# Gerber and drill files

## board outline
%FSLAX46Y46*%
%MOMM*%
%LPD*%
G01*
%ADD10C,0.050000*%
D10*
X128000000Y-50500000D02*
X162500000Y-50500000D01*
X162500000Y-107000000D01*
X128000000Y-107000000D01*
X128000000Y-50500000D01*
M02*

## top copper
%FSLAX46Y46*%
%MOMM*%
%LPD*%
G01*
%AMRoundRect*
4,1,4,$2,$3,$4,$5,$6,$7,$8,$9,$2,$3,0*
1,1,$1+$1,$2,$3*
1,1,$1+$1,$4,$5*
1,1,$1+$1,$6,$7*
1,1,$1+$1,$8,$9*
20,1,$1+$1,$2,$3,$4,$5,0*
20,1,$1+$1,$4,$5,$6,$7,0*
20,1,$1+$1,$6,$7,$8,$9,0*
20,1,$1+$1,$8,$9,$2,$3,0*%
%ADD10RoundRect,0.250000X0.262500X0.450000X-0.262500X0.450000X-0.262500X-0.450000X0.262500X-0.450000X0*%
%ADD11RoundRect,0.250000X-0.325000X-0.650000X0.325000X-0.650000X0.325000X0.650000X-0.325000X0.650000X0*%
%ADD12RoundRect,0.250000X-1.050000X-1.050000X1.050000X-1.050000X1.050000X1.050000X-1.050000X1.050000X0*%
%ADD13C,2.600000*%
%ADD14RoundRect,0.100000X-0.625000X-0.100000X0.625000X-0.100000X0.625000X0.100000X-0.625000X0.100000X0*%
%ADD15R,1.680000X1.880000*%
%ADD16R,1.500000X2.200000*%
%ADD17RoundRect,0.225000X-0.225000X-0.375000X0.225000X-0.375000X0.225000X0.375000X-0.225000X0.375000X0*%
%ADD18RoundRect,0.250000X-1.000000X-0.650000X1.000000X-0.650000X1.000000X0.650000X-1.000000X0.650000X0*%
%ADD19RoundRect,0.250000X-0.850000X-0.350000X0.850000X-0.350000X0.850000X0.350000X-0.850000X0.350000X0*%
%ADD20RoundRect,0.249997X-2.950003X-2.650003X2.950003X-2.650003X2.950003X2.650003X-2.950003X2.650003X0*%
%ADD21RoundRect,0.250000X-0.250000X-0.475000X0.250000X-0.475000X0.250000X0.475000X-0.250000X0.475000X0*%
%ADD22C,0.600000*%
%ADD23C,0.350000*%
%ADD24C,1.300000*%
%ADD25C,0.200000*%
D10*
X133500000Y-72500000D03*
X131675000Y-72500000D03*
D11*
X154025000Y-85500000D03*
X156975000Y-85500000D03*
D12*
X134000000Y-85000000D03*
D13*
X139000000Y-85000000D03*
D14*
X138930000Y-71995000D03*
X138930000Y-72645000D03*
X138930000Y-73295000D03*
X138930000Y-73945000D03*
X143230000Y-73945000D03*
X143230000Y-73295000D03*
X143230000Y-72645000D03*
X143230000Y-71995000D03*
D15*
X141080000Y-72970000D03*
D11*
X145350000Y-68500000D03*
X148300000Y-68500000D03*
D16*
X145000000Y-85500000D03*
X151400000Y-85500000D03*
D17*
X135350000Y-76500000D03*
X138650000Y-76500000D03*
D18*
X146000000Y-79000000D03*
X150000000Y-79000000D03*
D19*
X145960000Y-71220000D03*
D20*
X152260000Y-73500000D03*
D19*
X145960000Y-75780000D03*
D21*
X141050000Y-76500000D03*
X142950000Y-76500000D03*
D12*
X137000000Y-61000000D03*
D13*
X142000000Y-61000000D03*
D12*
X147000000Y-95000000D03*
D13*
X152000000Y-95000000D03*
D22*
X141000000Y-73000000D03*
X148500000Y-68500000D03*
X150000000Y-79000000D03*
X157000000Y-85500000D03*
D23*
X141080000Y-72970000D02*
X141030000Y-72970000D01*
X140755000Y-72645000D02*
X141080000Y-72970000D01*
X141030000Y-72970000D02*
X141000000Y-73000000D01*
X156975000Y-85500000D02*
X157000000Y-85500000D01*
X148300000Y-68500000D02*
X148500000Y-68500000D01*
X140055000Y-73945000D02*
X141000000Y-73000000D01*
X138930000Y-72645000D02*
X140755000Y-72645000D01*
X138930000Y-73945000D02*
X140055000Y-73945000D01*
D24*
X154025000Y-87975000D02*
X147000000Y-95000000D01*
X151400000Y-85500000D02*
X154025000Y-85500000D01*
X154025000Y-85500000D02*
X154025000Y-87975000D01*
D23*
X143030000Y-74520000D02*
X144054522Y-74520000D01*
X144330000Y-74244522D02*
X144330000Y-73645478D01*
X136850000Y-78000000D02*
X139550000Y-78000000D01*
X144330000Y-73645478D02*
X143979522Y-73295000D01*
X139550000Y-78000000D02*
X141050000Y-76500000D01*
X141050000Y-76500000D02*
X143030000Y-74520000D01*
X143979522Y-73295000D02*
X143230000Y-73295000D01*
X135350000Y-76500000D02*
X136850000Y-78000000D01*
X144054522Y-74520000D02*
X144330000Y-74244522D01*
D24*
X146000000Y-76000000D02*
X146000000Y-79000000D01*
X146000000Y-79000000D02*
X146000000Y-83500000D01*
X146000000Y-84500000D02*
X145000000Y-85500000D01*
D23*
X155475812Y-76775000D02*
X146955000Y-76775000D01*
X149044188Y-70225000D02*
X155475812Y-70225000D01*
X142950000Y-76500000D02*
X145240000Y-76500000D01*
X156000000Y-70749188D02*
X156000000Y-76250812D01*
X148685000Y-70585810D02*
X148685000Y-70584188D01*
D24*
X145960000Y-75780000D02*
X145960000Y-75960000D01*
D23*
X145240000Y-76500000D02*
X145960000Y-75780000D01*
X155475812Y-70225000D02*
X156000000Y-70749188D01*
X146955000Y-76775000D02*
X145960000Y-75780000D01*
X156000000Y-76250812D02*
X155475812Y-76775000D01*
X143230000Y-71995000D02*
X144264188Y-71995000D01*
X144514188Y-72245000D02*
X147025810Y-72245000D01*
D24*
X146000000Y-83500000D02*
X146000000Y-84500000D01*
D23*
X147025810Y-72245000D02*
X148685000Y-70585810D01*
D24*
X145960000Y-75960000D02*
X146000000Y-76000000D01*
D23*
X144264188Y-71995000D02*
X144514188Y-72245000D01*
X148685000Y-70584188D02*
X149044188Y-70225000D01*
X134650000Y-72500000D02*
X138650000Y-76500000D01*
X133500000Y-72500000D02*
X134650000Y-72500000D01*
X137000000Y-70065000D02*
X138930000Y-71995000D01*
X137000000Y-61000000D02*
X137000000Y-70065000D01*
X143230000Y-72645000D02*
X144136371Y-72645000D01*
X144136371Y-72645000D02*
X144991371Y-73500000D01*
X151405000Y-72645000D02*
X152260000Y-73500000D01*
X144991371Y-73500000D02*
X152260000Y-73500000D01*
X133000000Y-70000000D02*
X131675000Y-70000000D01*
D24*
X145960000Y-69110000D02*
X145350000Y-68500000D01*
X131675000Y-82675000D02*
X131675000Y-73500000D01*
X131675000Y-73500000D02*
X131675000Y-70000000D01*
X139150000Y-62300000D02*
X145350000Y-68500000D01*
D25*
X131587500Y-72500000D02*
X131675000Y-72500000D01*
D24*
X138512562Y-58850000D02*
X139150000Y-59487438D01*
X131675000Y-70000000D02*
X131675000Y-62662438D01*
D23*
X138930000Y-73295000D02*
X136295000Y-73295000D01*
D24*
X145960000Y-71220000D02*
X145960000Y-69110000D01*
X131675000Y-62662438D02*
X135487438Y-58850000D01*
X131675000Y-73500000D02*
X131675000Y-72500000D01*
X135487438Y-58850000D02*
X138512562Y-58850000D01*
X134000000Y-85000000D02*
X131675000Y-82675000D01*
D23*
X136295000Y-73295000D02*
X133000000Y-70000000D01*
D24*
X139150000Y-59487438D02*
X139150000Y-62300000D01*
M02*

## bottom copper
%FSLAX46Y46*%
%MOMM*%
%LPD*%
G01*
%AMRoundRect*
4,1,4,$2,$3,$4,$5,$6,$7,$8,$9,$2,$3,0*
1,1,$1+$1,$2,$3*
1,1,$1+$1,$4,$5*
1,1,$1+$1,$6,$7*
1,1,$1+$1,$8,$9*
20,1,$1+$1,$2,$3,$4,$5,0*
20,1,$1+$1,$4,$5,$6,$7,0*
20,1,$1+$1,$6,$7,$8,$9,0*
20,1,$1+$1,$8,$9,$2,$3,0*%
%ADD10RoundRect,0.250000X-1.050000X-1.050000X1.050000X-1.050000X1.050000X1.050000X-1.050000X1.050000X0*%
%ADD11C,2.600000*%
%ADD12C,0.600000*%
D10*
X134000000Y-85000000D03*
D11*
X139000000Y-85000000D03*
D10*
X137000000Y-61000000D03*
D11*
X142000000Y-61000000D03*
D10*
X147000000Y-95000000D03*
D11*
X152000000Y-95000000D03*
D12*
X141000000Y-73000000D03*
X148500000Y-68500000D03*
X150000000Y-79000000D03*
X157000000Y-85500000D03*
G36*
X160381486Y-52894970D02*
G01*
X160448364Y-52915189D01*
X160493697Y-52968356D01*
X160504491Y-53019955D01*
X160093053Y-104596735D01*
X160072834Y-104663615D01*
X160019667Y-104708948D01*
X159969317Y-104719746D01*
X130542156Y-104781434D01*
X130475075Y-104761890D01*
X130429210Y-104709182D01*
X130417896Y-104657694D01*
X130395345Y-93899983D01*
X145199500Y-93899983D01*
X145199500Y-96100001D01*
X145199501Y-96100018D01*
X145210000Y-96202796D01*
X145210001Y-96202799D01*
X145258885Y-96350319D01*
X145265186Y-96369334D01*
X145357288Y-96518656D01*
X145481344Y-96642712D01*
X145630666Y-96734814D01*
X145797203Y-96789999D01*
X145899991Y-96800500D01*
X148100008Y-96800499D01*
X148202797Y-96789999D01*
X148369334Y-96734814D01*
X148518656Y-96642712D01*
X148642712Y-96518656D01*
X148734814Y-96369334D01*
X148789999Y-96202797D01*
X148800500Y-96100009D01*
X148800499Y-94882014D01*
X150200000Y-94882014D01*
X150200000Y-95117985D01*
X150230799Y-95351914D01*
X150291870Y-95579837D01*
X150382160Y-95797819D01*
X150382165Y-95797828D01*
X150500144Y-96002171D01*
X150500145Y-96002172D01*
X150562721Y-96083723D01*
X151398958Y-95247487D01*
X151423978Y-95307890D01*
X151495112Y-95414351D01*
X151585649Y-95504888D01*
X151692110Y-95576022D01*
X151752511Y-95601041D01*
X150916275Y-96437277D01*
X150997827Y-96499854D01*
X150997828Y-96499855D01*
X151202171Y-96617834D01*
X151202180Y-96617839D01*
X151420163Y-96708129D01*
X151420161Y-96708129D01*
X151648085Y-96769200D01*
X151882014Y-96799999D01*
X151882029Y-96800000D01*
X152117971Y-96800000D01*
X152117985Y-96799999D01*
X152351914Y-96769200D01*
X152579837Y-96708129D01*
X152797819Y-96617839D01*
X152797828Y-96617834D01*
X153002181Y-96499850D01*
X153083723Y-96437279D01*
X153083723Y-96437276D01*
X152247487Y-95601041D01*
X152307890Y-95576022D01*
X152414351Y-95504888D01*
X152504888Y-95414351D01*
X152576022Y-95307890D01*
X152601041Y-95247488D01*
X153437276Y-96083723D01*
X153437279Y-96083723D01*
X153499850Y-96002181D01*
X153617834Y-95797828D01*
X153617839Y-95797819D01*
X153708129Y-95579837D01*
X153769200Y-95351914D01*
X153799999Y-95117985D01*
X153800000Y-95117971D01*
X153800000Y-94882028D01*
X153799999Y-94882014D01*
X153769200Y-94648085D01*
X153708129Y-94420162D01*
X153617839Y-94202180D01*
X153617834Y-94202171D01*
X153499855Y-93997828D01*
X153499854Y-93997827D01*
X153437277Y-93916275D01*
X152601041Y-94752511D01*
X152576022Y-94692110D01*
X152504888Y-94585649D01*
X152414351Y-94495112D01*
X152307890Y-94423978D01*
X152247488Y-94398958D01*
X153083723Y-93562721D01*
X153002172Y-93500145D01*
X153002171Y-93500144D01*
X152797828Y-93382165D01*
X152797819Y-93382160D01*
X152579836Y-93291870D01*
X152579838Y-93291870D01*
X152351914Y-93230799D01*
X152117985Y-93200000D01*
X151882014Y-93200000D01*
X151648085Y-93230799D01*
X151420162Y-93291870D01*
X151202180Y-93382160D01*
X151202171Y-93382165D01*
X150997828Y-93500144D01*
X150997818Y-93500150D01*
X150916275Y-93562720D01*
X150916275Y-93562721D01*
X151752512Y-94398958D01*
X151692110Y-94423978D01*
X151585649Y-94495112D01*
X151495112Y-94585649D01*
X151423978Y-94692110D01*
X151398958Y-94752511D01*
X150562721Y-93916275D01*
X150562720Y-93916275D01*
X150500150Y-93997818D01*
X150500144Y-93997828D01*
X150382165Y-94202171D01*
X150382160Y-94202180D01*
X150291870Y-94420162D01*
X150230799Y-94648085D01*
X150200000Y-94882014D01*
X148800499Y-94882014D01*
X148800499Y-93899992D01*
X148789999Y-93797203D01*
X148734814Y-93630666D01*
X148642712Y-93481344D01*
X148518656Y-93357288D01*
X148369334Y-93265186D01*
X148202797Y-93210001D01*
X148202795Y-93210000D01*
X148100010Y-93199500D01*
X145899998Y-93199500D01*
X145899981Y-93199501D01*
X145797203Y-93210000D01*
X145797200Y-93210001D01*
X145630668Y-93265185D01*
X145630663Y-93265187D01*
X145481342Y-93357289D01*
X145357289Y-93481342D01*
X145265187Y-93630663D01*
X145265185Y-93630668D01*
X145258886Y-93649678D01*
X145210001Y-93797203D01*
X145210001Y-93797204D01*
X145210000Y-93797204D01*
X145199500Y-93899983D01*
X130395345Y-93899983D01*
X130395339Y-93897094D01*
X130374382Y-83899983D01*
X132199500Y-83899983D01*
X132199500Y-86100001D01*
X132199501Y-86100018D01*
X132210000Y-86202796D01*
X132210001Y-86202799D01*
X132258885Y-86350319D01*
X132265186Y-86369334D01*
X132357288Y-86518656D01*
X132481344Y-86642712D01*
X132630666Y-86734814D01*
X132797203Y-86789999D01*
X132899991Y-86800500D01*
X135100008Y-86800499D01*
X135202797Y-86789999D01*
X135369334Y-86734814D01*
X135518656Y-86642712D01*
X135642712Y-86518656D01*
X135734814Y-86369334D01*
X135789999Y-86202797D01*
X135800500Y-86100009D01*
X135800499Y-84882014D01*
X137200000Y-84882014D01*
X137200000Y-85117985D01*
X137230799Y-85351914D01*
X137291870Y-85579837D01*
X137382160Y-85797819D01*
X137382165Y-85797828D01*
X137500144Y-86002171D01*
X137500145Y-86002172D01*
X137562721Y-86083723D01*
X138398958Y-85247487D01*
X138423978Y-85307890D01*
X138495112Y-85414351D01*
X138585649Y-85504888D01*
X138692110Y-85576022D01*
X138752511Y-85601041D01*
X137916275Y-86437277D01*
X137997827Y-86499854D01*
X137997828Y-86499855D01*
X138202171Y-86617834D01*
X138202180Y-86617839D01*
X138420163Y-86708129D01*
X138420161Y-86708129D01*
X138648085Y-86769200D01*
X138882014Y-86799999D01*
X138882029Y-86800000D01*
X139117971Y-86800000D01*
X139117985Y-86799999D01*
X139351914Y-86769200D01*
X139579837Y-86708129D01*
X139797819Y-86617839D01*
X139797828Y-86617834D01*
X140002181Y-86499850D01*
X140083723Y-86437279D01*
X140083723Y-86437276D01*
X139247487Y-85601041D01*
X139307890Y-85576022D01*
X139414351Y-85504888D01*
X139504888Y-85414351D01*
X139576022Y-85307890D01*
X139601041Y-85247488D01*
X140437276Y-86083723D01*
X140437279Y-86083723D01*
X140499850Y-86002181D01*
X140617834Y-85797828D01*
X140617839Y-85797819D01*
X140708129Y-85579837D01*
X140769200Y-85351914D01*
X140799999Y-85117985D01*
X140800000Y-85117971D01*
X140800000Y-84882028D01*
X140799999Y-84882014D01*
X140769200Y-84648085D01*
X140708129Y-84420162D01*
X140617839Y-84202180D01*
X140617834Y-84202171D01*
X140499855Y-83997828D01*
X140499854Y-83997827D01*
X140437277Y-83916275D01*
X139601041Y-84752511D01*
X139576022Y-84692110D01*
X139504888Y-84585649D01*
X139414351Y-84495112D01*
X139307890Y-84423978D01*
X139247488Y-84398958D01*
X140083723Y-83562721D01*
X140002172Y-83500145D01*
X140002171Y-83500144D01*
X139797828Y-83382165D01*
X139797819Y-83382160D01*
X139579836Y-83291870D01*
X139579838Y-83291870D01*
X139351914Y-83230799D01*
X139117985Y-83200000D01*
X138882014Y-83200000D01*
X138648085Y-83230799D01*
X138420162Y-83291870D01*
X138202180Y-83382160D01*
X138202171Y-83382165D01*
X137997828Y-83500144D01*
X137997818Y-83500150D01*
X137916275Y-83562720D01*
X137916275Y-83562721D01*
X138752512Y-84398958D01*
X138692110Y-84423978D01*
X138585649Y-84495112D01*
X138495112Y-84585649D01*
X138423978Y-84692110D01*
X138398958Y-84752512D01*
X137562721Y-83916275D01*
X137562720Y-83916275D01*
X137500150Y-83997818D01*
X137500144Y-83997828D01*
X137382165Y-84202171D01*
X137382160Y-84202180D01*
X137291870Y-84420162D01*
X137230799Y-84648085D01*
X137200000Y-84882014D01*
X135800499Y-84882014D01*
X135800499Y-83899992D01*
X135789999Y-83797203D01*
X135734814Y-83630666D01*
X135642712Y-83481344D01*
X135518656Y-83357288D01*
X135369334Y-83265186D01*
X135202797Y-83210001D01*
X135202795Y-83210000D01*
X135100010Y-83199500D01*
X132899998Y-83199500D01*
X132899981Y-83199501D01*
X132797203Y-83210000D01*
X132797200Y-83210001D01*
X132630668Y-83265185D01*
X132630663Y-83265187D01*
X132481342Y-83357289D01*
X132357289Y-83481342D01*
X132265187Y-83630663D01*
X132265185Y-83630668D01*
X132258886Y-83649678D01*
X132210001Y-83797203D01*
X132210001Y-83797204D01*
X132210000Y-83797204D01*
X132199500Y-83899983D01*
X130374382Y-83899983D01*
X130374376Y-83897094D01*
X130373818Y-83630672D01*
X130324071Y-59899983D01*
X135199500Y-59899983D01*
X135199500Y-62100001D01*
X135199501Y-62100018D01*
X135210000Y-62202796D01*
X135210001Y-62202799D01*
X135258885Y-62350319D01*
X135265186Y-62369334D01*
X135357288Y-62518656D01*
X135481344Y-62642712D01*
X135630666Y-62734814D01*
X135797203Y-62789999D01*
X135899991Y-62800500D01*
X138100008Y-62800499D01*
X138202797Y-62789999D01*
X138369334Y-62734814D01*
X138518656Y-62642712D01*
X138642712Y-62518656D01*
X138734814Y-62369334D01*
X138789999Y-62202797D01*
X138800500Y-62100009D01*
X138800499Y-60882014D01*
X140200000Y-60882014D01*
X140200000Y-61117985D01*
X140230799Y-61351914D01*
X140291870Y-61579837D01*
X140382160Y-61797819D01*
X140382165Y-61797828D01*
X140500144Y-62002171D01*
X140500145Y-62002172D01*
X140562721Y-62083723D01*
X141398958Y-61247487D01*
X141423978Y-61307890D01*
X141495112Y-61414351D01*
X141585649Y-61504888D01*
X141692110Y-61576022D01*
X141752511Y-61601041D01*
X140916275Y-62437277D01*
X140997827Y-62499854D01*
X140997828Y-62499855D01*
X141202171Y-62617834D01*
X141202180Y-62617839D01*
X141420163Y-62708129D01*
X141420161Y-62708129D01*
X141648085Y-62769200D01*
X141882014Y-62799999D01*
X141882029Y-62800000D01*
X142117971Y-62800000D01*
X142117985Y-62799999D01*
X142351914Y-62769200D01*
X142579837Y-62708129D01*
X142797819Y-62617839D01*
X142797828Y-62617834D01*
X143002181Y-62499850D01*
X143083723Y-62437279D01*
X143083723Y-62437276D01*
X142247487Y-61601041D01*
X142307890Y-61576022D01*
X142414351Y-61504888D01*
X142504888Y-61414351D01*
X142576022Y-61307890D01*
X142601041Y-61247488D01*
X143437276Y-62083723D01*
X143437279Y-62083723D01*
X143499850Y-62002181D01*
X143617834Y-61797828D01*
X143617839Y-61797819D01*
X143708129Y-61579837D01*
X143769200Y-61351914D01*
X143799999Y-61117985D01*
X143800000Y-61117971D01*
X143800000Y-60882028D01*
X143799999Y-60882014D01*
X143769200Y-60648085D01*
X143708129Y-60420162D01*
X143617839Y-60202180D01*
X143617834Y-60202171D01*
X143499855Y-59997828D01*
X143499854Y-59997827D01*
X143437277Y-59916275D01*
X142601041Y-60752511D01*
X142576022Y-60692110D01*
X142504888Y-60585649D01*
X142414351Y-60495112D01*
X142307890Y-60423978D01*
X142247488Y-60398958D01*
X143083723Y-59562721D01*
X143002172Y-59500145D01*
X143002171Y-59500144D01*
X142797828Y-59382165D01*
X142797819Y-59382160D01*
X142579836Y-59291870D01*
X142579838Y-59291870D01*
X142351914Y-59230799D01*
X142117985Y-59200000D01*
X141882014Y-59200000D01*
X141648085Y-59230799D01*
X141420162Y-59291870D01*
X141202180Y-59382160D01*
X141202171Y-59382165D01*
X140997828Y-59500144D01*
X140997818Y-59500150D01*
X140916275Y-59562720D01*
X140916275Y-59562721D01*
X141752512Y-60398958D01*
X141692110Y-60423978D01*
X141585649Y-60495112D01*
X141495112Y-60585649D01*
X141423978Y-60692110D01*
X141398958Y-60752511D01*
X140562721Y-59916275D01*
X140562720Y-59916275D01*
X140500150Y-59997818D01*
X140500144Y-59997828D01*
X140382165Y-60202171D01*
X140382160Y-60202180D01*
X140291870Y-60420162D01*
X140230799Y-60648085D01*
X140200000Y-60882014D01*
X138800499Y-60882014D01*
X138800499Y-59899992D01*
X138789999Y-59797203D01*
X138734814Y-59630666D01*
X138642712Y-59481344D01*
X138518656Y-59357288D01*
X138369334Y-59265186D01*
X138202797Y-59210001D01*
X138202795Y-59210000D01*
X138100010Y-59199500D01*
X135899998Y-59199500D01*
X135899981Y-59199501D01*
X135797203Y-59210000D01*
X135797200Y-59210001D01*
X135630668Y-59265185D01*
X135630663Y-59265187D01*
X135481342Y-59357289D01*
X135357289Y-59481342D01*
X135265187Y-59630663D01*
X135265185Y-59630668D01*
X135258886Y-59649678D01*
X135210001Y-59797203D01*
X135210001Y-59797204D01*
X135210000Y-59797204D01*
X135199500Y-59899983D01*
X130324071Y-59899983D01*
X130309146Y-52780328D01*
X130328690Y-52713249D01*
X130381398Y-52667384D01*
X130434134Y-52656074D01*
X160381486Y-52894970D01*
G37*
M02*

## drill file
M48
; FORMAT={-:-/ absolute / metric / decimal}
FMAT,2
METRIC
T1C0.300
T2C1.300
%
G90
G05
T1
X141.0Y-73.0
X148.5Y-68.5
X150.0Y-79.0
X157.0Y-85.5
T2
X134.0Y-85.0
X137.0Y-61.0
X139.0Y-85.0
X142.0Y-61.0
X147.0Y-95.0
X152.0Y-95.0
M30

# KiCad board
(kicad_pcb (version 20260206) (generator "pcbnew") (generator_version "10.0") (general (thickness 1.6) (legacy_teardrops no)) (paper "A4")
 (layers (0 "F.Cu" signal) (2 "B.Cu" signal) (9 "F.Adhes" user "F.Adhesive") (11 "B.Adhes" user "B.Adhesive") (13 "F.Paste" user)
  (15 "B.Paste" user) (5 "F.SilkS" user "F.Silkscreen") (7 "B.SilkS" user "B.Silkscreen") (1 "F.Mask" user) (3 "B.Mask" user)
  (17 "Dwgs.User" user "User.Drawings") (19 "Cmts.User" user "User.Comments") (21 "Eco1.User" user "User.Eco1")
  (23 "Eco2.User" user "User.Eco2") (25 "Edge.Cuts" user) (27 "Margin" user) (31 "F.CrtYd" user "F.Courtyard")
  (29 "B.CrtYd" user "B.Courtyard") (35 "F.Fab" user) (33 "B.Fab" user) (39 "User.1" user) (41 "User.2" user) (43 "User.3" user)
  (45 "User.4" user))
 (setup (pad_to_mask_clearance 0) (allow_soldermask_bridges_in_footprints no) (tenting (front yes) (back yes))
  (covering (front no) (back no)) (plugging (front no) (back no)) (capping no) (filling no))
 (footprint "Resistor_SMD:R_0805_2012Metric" (layer "F.Cu") (at 132.5875 72.5 180)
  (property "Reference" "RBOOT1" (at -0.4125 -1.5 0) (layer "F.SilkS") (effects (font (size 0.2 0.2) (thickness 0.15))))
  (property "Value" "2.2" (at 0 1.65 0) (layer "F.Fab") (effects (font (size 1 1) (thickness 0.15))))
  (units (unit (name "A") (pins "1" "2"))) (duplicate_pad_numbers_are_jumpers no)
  (pad "1" smd roundrect (at -0.9125 0 180) (size 1.025 1.4) (layers "F.Cu" "F.Mask" "F.Paste") (roundrect_rratio 0.243902)
   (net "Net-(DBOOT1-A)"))
  (pad "2" smd roundrect (at 0.9125 0 180) (size 1.025 1.4) (layers "F.Cu" "F.Mask" "F.Paste") (roundrect_rratio 0.243902) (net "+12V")))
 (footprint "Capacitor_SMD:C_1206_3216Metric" (layer "F.Cu") (at 155.5 85.5)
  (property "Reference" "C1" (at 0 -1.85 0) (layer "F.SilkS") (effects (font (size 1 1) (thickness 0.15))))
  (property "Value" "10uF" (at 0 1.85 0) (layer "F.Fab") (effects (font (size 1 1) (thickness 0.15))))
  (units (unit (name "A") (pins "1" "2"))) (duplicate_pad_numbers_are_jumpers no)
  (pad "1" smd roundrect (at -1.475 0) (size 1.15 1.8) (layers "F.Cu" "F.Mask" "F.Paste") (roundrect_rratio 0.217391)
   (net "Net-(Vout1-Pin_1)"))
  (pad "2" smd roundrect (at 1.475 0) (size 1.15 1.8) (layers "F.Cu" "F.Mask" "F.Paste") (roundrect_rratio 0.217391) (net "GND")))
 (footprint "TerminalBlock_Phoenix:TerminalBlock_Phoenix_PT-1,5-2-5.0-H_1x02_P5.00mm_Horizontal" (layer "F.Cu") (at 134 85)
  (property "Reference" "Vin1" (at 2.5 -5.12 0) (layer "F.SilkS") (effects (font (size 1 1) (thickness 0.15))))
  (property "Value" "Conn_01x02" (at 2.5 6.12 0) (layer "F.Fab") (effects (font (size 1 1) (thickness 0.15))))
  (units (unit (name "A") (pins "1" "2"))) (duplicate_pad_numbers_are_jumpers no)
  (pad "1" thru_hole roundrect (at 0 0) (size 2.6 2.6) (drill 1.3) (layers "*.Cu" "*.Mask") (remove_unused_layers no)
   (roundrect_rratio 0.096154) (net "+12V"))
  (pad "2" thru_hole circle (at 5 0) (size 2.6 2.6) (drill 1.3) (layers "*.Cu" "*.Mask") (remove_unused_layers no) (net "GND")))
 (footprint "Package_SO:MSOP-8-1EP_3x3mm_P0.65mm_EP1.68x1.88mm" (layer "F.Cu") (at 141.08 72.97)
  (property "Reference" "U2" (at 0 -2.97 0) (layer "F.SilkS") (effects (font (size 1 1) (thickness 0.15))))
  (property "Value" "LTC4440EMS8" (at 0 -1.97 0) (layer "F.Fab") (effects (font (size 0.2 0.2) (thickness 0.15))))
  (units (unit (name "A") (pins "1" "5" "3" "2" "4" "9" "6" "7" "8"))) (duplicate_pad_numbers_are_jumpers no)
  (pad "" smd roundrect (at -0.42 -0.47) (size 0.68 0.76) (layers "F.Paste") (roundrect_rratio 0.25))
  (pad "" smd roundrect (at -0.42 0.47) (size 0.68 0.76) (layers "F.Paste") (roundrect_rratio 0.25))
  (pad "" smd roundrect (at 0.42 -0.47) (size 0.68 0.76) (layers "F.Paste") (roundrect_rratio 0.25))
  (pad "" smd roundrect (at 0.42 0.47) (size 0.68 0.76) (layers "F.Paste") (roundrect_rratio 0.25))
  (pad "1" smd roundrect (at -2.15 -0.975) (size 1.45 0.4) (layers "F.Cu" "F.Mask" "F.Paste") (roundrect_rratio 0.25)
   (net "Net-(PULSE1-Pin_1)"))
  (pad "2" smd roundrect (at -2.15 -0.325) (size 1.45 0.4) (layers "F.Cu" "F.Mask" "F.Paste") (roundrect_rratio 0.25) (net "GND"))
  (pad "3" smd roundrect (at -2.15 0.325) (size 1.45 0.4) (layers "F.Cu" "F.Mask" "F.Paste") (roundrect_rratio 0.25) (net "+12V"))
  (pad "4" smd roundrect (at -2.15 0.975) (size 1.45 0.4) (layers "F.Cu" "F.Mask" "F.Paste") (roundrect_rratio 0.25) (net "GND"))
  (pad "5" smd roundrect (at 2.15 0.975) (size 1.45 0.4) (layers "F.Cu" "F.Mask" "F.Paste") (roundrect_rratio 0.25)
   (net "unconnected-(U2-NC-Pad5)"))
  (pad "6" smd roundrect (at 2.15 0.325) (size 1.45 0.4) (layers "F.Cu" "F.Mask" "F.Paste") (roundrect_rratio 0.25) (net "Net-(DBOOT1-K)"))
  (pad "7" smd roundrect (at 2.15 -0.325) (size 1.45 0.4) (layers "F.Cu" "F.Mask" "F.Paste") (roundrect_rratio 0.25) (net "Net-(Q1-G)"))
  (pad "8" smd roundrect (at 2.15 -0.975) (size 1.45 0.4) (layers "F.Cu" "F.Mask" "F.Paste") (roundrect_rratio 0.25) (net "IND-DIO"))
  (pad "9" smd rect (at 0 0) (size 1.68 1.88) (layers "F.Cu" "F.Mask") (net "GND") (zone_connect 2)))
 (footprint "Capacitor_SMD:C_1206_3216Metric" (layer "F.Cu") (at 146.825 68.5)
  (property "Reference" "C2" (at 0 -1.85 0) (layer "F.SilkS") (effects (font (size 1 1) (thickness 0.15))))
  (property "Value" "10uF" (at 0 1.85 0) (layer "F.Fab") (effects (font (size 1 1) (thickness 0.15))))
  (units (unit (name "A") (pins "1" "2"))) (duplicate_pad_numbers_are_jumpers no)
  (pad "1" smd roundrect (at -1.475 0) (size 1.15 1.8) (layers "F.Cu" "F.Mask" "F.Paste") (roundrect_rratio 0.217391) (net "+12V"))
  (pad "2" smd roundrect (at 1.475 0) (size 1.15 1.8) (layers "F.Cu" "F.Mask" "F.Paste") (roundrect_rratio 0.217391) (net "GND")))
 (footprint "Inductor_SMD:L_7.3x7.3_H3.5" (layer "F.Cu") (at 148.2 85.5)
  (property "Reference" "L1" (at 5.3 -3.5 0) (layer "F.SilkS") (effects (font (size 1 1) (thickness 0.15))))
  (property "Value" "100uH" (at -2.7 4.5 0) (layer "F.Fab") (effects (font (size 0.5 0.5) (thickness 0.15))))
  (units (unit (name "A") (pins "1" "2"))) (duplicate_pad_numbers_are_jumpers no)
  (pad "1" smd rect (at -3.2 0) (size 1.5 2.2) (layers "F.Cu" "F.Mask" "F.Paste") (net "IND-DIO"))
  (pad "2" smd rect (at 3.2 0) (size 1.5 2.2) (layers "F.Cu" "F.Mask" "F.Paste") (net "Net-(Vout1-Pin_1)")))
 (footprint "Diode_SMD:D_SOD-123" (layer "F.Cu") (at 137 76.5)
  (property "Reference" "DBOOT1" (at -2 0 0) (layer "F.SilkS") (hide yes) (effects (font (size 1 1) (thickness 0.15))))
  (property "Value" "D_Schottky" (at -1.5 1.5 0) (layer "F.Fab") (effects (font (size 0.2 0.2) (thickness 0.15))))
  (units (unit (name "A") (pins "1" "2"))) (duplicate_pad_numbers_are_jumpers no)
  (pad "1" smd roundrect (at -1.65 0) (size 0.9 1.2) (layers "F.Cu" "F.Mask" "F.Paste") (roundrect_rratio 0.25) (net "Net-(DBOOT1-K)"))
  (pad "2" smd roundrect (at 1.65 0) (size 0.9 1.2) (layers "F.Cu" "F.Mask" "F.Paste") (roundrect_rratio 0.25) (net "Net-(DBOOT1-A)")))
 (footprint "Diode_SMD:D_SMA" (layer "F.Cu") (at 148 79)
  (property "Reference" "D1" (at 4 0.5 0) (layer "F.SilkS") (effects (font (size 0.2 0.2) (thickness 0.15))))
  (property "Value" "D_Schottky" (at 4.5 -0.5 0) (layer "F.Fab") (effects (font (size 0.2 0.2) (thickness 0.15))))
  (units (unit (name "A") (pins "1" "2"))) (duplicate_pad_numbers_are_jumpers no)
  (pad "1" smd roundrect (at -2 0) (size 2.5 1.8) (layers "F.Cu" "F.Mask" "F.Paste") (roundrect_rratio 0.1388888889) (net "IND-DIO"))
  (pad "2" smd roundrect (at 2 0) (size 2.5 1.8) (layers "F.Cu" "F.Mask" "F.Paste") (roundrect_rratio 0.1388888889) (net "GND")))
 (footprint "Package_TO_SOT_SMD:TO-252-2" (layer "F.Cu") (at 151 73.5)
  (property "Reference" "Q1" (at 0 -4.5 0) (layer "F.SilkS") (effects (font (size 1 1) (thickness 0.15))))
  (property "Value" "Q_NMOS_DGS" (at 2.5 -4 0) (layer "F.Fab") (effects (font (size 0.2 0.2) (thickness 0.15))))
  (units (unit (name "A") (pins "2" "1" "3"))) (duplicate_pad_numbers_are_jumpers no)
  (pad "" smd roundrect (at -0.415 -1.525) (size 3.05 2.75) (layers "F.Paste") (roundrect_rratio 0.090909))
  (pad "" smd roundrect (at -0.415 1.525) (size 3.05 2.75) (layers "F.Paste") (roundrect_rratio 0.090909))
  (pad "" smd roundrect (at 2.935 -1.525) (size 3.05 2.75) (layers "F.Paste") (roundrect_rratio 0.090909))
  (pad "" smd roundrect (at 2.935 1.525) (size 3.05 2.75) (layers "F.Paste") (roundrect_rratio 0.090909))
  (pad "1" smd roundrect (at -5.04 -2.28) (size 2.2 1.2) (layers "F.Cu" "F.Mask" "F.Paste") (roundrect_rratio 0.208333) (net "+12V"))
  (pad "2" smd roundrect (at 1.26 0) (size 6.4 5.8) (layers "F.Cu" "F.Mask") (roundrect_rratio 0.043103) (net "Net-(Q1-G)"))
  (pad "3" smd roundrect (at -5.04 2.28) (size 2.2 1.2) (layers "F.Cu" "F.Mask" "F.Paste") (roundrect_rratio 0.208333) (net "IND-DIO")))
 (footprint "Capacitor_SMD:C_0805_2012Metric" (layer "F.Cu") (at 142 76.5)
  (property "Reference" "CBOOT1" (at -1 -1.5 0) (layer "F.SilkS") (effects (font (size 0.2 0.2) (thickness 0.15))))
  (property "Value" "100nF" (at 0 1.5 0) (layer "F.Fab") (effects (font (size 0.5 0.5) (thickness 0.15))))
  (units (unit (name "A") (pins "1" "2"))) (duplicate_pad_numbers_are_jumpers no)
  (pad "1" smd roundrect (at -0.95 0) (size 1 1.45) (layers "F.Cu" "F.Mask" "F.Paste") (roundrect_rratio 0.25) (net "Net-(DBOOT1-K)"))
  (pad "2" smd roundrect (at 0.95 0) (size 1 1.45) (layers "F.Cu" "F.Mask" "F.Paste") (roundrect_rratio 0.25) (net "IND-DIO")))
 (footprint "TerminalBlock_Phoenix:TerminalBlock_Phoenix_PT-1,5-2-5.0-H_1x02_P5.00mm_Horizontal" (layer "F.Cu") (at 137 61)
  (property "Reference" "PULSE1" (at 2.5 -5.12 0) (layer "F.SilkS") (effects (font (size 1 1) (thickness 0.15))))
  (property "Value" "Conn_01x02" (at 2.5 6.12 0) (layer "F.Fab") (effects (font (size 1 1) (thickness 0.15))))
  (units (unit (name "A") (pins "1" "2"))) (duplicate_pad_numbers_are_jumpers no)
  (pad "1" thru_hole roundrect (at 0 0) (size 2.6 2.6) (drill 1.3) (layers "*.Cu" "*.Mask") (remove_unused_layers no)
   (roundrect_rratio 0.096154) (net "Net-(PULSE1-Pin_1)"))
  (pad "2" thru_hole circle (at 5 0) (size 2.6 2.6) (drill 1.3) (layers "*.Cu" "*.Mask") (remove_unused_layers no) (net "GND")))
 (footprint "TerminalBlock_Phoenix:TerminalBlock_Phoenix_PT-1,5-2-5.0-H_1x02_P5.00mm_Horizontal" (layer "F.Cu") (at 147 95)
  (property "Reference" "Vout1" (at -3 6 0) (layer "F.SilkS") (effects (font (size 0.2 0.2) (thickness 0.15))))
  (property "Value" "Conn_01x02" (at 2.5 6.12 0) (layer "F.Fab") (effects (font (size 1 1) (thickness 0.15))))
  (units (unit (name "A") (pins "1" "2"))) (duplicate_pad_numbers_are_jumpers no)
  (pad "1" thru_hole roundrect (at 0 0) (size 2.6 2.6) (drill 1.3) (layers "*.Cu" "*.Mask") (remove_unused_layers no)
   (roundrect_rratio 0.096154) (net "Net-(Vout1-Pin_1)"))
  (pad "2" thru_hole circle (at 5 0) (size 2.6 2.6) (drill 1.3) (layers "*.Cu" "*.Mask") (remove_unused_layers no) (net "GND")))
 (gr_rect (start 128 50.5) (end 162.5 107) (stroke (width 0.05) (type default)) (fill no) (layer "Edge.Cuts"))
 (segment (start 141.08 72.97) (end 141.03 72.97) (width 0.35) (layer "F.Cu") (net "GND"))
 (segment (start 140.755 72.645) (end 141.08 72.97) (width 0.35) (layer "F.Cu") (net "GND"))
 (segment (start 141.03 72.97) (end 141 73) (width 0.35) (layer "F.Cu") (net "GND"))
 (segment (start 156.975 85.5) (end 157 85.5) (width 0.35) (layer "F.Cu") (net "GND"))
 (segment (start 148.3 68.5) (end 148.5 68.5) (width 0.35) (layer "F.Cu") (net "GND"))
 (segment (start 140.055 73.945) (end 141 73) (width 0.35) (layer "F.Cu") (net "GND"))
 (segment (start 138.93 72.645) (end 140.755 72.645) (width 0.35) (layer "F.Cu") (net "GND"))
 (segment (start 138.93 73.945) (end 140.055 73.945) (width 0.35) (layer "F.Cu") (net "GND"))
 (via (at 141 73) (size 0.6) (drill 0.3) (layers "F.Cu" "B.Cu") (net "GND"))
 (via (at 148.5 68.5) (size 0.6) (drill 0.3) (layers "F.Cu" "B.Cu") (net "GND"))
 (via (at 150 79) (size 0.6) (drill 0.3) (layers "F.Cu" "B.Cu") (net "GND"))
 (via (at 157 85.5) (size 0.6) (drill 0.3) (layers "F.Cu" "B.Cu") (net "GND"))
 (segment (start 154.025 87.975) (end 147 95) (width 1.3) (layer "F.Cu") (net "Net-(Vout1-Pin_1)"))
 (segment (start 151.4 85.5) (end 154.025 85.5) (width 1.3) (layer "F.Cu") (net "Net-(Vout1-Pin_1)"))
 (segment (start 154.025 85.5) (end 154.025 87.975) (width 1.3) (layer "F.Cu") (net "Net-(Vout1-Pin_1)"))
 (segment (start 143.03 74.52) (end 144.054522 74.52) (width 0.35) (layer "F.Cu") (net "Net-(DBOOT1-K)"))
 (segment (start 144.33 74.244522) (end 144.33 73.645478) (width 0.35) (layer "F.Cu") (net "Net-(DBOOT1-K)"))
 (segment (start 136.85 78) (end 139.55 78) (width 0.35) (layer "F.Cu") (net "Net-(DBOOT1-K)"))
 (segment (start 144.33 73.645478) (end 143.979522 73.295) (width 0.35) (layer "F.Cu") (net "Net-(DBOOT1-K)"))
 (segment (start 139.55 78) (end 141.05 76.5) (width 0.35) (layer "F.Cu") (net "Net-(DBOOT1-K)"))
 (segment (start 141.05 76.5) (end 143.03 74.52) (width 0.35) (layer "F.Cu") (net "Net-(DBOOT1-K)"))
 (segment (start 143.979522 73.295) (end 143.23 73.295) (width 0.35) (layer "F.Cu") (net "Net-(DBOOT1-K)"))
 (segment (start 135.35 76.5) (end 136.85 78) (width 0.35) (layer "F.Cu") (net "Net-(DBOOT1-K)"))
 (segment (start 144.054522 74.52) (end 144.33 74.244522) (width 0.35) (layer "F.Cu") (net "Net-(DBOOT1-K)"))
 (segment (start 146 76) (end 146 79) (width 1.3) (layer "F.Cu") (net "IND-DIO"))
 (segment (start 146 79) (end 146 83.5) (width 1.3) (layer "F.Cu") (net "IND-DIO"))
 (segment (start 146 84.5) (end 145 85.5) (width 1.3) (layer "F.Cu") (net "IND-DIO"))
 (segment (start 155.475812 76.775) (end 146.955 76.775) (width 0.35) (layer "F.Cu") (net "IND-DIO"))
 (segment (start 149.044188 70.225) (end 155.475812 70.225) (width 0.35) (layer "F.Cu") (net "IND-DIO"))
 (segment (start 142.95 76.5) (end 145.24 76.5) (width 0.35) (layer "F.Cu") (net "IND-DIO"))
 (segment (start 156 70.749188) (end 156 76.250812) (width 0.35) (layer "F.Cu") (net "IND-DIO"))
 (segment (start 148.685 70.58581) (end 148.685 70.584188) (width 0.35) (layer "F.Cu") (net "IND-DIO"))
 (segment (start 145.96 75.78) (end 145.96 75.96) (width 1.3) (layer "F.Cu") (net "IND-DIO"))
 (segment (start 145.24 76.5) (end 145.96 75.78) (width 0.35) (layer "F.Cu") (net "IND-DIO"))
 (segment (start 155.475812 70.225) (end 156 70.749188) (width 0.35) (layer "F.Cu") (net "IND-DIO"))
 (segment (start 146.955 76.775) (end 145.96 75.78) (width 0.35) (layer "F.Cu") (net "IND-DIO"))
 (segment (start 156 76.250812) (end 155.475812 76.775) (width 0.35) (layer "F.Cu") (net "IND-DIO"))
 (segment (start 143.23 71.995) (end 144.264188 71.995) (width 0.35) (layer "F.Cu") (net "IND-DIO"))
 (segment (start 144.514188 72.245) (end 147.02581 72.245) (width 0.35) (layer "F.Cu") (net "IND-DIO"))
 (segment (start 146 83.5) (end 146 84.5) (width 1.3) (layer "F.Cu") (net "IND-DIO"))
 (segment (start 147.02581 72.245) (end 148.685 70.58581) (width 0.35) (layer "F.Cu") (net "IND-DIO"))
 (segment (start 145.96 75.96) (end 146 76) (width 1.3) (layer "F.Cu") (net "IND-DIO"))
 (segment (start 144.264188 71.995) (end 144.514188 72.245) (width 0.35) (layer "F.Cu") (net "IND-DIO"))
 (segment (start 148.685 70.584188) (end 149.044188 70.225) (width 0.35) (layer "F.Cu") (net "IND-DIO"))
 (segment (start 134.65 72.5) (end 138.65 76.5) (width 0.35) (layer "F.Cu") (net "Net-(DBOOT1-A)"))
 (segment (start 133.5 72.5) (end 134.65 72.5) (width 0.35) (layer "F.Cu") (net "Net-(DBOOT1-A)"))
 (segment (start 137 70.065) (end 138.93 71.995) (width 0.35) (layer "F.Cu") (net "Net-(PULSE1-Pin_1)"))
 (segment (start 137 61) (end 137 70.065) (width 0.35) (layer "F.Cu") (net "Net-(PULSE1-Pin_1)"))
 (segment (start 143.23 72.645) (end 144.136371 72.645) (width 0.35) (layer "F.Cu") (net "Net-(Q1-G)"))
 (segment (start 144.136371 72.645) (end 144.991371 73.5) (width 0.35) (layer "F.Cu") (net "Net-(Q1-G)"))
 (segment (start 151.405 72.645) (end 152.26 73.5) (width 0.35) (layer "F.Cu") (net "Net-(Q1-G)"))
 (segment (start 144.991371 73.5) (end 152.26 73.5) (width 0.35) (layer "F.Cu") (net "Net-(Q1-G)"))
 (segment (start 133 70) (end 131.675 70) (width 0.35) (layer "F.Cu") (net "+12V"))
 (segment (start 145.96 69.11) (end 145.35 68.5) (width 1.3) (layer "F.Cu") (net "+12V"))
 (segment (start 131.675 82.675) (end 131.675 73.5) (width 1.3) (layer "F.Cu") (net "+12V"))
 (segment (start 131.675 73.5) (end 131.675 70) (width 1.3) (layer "F.Cu") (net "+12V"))
 (segment (start 139.15 62.3) (end 145.35 68.5) (width 1.3) (layer "F.Cu") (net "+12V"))
 (segment (start 131.5875 72.5) (end 131.675 72.5) (width 0.2) (layer "F.Cu") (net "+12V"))
 (segment (start 138.512562 58.85) (end 139.15 59.487438) (width 1.3) (layer "F.Cu") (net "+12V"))
 (segment (start 131.675 70) (end 131.675 62.662438) (width 1.3) (layer "F.Cu") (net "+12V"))
 (segment (start 138.93 73.295) (end 136.295 73.295) (width 0.35) (layer "F.Cu") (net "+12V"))
 (segment (start 145.96 71.22) (end 145.96 69.11) (width 1.3) (layer "F.Cu") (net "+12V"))
 (segment (start 131.675 62.662438) (end 135.487438 58.85) (width 1.3) (layer "F.Cu") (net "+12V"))
 (segment (start 131.675 73.5) (end 131.675 72.5) (width 1.3) (layer "F.Cu") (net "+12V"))
 (segment (start 135.487438 58.85) (end 138.512562 58.85) (width 1.3) (layer "F.Cu") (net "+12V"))
 (segment (start 134 85) (end 131.675 82.675) (width 1.3) (layer "F.Cu") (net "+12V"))
 (segment (start 136.295 73.295) (end 133 70) (width 0.35) (layer "F.Cu") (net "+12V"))
 (segment (start 139.15 59.487438) (end 139.15 62.3) (width 1.3) (layer "F.Cu") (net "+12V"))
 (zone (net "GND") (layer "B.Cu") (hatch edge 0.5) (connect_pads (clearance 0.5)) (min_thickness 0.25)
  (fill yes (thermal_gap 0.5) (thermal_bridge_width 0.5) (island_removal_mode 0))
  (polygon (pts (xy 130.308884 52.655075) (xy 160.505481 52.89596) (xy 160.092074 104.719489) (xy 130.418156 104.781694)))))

